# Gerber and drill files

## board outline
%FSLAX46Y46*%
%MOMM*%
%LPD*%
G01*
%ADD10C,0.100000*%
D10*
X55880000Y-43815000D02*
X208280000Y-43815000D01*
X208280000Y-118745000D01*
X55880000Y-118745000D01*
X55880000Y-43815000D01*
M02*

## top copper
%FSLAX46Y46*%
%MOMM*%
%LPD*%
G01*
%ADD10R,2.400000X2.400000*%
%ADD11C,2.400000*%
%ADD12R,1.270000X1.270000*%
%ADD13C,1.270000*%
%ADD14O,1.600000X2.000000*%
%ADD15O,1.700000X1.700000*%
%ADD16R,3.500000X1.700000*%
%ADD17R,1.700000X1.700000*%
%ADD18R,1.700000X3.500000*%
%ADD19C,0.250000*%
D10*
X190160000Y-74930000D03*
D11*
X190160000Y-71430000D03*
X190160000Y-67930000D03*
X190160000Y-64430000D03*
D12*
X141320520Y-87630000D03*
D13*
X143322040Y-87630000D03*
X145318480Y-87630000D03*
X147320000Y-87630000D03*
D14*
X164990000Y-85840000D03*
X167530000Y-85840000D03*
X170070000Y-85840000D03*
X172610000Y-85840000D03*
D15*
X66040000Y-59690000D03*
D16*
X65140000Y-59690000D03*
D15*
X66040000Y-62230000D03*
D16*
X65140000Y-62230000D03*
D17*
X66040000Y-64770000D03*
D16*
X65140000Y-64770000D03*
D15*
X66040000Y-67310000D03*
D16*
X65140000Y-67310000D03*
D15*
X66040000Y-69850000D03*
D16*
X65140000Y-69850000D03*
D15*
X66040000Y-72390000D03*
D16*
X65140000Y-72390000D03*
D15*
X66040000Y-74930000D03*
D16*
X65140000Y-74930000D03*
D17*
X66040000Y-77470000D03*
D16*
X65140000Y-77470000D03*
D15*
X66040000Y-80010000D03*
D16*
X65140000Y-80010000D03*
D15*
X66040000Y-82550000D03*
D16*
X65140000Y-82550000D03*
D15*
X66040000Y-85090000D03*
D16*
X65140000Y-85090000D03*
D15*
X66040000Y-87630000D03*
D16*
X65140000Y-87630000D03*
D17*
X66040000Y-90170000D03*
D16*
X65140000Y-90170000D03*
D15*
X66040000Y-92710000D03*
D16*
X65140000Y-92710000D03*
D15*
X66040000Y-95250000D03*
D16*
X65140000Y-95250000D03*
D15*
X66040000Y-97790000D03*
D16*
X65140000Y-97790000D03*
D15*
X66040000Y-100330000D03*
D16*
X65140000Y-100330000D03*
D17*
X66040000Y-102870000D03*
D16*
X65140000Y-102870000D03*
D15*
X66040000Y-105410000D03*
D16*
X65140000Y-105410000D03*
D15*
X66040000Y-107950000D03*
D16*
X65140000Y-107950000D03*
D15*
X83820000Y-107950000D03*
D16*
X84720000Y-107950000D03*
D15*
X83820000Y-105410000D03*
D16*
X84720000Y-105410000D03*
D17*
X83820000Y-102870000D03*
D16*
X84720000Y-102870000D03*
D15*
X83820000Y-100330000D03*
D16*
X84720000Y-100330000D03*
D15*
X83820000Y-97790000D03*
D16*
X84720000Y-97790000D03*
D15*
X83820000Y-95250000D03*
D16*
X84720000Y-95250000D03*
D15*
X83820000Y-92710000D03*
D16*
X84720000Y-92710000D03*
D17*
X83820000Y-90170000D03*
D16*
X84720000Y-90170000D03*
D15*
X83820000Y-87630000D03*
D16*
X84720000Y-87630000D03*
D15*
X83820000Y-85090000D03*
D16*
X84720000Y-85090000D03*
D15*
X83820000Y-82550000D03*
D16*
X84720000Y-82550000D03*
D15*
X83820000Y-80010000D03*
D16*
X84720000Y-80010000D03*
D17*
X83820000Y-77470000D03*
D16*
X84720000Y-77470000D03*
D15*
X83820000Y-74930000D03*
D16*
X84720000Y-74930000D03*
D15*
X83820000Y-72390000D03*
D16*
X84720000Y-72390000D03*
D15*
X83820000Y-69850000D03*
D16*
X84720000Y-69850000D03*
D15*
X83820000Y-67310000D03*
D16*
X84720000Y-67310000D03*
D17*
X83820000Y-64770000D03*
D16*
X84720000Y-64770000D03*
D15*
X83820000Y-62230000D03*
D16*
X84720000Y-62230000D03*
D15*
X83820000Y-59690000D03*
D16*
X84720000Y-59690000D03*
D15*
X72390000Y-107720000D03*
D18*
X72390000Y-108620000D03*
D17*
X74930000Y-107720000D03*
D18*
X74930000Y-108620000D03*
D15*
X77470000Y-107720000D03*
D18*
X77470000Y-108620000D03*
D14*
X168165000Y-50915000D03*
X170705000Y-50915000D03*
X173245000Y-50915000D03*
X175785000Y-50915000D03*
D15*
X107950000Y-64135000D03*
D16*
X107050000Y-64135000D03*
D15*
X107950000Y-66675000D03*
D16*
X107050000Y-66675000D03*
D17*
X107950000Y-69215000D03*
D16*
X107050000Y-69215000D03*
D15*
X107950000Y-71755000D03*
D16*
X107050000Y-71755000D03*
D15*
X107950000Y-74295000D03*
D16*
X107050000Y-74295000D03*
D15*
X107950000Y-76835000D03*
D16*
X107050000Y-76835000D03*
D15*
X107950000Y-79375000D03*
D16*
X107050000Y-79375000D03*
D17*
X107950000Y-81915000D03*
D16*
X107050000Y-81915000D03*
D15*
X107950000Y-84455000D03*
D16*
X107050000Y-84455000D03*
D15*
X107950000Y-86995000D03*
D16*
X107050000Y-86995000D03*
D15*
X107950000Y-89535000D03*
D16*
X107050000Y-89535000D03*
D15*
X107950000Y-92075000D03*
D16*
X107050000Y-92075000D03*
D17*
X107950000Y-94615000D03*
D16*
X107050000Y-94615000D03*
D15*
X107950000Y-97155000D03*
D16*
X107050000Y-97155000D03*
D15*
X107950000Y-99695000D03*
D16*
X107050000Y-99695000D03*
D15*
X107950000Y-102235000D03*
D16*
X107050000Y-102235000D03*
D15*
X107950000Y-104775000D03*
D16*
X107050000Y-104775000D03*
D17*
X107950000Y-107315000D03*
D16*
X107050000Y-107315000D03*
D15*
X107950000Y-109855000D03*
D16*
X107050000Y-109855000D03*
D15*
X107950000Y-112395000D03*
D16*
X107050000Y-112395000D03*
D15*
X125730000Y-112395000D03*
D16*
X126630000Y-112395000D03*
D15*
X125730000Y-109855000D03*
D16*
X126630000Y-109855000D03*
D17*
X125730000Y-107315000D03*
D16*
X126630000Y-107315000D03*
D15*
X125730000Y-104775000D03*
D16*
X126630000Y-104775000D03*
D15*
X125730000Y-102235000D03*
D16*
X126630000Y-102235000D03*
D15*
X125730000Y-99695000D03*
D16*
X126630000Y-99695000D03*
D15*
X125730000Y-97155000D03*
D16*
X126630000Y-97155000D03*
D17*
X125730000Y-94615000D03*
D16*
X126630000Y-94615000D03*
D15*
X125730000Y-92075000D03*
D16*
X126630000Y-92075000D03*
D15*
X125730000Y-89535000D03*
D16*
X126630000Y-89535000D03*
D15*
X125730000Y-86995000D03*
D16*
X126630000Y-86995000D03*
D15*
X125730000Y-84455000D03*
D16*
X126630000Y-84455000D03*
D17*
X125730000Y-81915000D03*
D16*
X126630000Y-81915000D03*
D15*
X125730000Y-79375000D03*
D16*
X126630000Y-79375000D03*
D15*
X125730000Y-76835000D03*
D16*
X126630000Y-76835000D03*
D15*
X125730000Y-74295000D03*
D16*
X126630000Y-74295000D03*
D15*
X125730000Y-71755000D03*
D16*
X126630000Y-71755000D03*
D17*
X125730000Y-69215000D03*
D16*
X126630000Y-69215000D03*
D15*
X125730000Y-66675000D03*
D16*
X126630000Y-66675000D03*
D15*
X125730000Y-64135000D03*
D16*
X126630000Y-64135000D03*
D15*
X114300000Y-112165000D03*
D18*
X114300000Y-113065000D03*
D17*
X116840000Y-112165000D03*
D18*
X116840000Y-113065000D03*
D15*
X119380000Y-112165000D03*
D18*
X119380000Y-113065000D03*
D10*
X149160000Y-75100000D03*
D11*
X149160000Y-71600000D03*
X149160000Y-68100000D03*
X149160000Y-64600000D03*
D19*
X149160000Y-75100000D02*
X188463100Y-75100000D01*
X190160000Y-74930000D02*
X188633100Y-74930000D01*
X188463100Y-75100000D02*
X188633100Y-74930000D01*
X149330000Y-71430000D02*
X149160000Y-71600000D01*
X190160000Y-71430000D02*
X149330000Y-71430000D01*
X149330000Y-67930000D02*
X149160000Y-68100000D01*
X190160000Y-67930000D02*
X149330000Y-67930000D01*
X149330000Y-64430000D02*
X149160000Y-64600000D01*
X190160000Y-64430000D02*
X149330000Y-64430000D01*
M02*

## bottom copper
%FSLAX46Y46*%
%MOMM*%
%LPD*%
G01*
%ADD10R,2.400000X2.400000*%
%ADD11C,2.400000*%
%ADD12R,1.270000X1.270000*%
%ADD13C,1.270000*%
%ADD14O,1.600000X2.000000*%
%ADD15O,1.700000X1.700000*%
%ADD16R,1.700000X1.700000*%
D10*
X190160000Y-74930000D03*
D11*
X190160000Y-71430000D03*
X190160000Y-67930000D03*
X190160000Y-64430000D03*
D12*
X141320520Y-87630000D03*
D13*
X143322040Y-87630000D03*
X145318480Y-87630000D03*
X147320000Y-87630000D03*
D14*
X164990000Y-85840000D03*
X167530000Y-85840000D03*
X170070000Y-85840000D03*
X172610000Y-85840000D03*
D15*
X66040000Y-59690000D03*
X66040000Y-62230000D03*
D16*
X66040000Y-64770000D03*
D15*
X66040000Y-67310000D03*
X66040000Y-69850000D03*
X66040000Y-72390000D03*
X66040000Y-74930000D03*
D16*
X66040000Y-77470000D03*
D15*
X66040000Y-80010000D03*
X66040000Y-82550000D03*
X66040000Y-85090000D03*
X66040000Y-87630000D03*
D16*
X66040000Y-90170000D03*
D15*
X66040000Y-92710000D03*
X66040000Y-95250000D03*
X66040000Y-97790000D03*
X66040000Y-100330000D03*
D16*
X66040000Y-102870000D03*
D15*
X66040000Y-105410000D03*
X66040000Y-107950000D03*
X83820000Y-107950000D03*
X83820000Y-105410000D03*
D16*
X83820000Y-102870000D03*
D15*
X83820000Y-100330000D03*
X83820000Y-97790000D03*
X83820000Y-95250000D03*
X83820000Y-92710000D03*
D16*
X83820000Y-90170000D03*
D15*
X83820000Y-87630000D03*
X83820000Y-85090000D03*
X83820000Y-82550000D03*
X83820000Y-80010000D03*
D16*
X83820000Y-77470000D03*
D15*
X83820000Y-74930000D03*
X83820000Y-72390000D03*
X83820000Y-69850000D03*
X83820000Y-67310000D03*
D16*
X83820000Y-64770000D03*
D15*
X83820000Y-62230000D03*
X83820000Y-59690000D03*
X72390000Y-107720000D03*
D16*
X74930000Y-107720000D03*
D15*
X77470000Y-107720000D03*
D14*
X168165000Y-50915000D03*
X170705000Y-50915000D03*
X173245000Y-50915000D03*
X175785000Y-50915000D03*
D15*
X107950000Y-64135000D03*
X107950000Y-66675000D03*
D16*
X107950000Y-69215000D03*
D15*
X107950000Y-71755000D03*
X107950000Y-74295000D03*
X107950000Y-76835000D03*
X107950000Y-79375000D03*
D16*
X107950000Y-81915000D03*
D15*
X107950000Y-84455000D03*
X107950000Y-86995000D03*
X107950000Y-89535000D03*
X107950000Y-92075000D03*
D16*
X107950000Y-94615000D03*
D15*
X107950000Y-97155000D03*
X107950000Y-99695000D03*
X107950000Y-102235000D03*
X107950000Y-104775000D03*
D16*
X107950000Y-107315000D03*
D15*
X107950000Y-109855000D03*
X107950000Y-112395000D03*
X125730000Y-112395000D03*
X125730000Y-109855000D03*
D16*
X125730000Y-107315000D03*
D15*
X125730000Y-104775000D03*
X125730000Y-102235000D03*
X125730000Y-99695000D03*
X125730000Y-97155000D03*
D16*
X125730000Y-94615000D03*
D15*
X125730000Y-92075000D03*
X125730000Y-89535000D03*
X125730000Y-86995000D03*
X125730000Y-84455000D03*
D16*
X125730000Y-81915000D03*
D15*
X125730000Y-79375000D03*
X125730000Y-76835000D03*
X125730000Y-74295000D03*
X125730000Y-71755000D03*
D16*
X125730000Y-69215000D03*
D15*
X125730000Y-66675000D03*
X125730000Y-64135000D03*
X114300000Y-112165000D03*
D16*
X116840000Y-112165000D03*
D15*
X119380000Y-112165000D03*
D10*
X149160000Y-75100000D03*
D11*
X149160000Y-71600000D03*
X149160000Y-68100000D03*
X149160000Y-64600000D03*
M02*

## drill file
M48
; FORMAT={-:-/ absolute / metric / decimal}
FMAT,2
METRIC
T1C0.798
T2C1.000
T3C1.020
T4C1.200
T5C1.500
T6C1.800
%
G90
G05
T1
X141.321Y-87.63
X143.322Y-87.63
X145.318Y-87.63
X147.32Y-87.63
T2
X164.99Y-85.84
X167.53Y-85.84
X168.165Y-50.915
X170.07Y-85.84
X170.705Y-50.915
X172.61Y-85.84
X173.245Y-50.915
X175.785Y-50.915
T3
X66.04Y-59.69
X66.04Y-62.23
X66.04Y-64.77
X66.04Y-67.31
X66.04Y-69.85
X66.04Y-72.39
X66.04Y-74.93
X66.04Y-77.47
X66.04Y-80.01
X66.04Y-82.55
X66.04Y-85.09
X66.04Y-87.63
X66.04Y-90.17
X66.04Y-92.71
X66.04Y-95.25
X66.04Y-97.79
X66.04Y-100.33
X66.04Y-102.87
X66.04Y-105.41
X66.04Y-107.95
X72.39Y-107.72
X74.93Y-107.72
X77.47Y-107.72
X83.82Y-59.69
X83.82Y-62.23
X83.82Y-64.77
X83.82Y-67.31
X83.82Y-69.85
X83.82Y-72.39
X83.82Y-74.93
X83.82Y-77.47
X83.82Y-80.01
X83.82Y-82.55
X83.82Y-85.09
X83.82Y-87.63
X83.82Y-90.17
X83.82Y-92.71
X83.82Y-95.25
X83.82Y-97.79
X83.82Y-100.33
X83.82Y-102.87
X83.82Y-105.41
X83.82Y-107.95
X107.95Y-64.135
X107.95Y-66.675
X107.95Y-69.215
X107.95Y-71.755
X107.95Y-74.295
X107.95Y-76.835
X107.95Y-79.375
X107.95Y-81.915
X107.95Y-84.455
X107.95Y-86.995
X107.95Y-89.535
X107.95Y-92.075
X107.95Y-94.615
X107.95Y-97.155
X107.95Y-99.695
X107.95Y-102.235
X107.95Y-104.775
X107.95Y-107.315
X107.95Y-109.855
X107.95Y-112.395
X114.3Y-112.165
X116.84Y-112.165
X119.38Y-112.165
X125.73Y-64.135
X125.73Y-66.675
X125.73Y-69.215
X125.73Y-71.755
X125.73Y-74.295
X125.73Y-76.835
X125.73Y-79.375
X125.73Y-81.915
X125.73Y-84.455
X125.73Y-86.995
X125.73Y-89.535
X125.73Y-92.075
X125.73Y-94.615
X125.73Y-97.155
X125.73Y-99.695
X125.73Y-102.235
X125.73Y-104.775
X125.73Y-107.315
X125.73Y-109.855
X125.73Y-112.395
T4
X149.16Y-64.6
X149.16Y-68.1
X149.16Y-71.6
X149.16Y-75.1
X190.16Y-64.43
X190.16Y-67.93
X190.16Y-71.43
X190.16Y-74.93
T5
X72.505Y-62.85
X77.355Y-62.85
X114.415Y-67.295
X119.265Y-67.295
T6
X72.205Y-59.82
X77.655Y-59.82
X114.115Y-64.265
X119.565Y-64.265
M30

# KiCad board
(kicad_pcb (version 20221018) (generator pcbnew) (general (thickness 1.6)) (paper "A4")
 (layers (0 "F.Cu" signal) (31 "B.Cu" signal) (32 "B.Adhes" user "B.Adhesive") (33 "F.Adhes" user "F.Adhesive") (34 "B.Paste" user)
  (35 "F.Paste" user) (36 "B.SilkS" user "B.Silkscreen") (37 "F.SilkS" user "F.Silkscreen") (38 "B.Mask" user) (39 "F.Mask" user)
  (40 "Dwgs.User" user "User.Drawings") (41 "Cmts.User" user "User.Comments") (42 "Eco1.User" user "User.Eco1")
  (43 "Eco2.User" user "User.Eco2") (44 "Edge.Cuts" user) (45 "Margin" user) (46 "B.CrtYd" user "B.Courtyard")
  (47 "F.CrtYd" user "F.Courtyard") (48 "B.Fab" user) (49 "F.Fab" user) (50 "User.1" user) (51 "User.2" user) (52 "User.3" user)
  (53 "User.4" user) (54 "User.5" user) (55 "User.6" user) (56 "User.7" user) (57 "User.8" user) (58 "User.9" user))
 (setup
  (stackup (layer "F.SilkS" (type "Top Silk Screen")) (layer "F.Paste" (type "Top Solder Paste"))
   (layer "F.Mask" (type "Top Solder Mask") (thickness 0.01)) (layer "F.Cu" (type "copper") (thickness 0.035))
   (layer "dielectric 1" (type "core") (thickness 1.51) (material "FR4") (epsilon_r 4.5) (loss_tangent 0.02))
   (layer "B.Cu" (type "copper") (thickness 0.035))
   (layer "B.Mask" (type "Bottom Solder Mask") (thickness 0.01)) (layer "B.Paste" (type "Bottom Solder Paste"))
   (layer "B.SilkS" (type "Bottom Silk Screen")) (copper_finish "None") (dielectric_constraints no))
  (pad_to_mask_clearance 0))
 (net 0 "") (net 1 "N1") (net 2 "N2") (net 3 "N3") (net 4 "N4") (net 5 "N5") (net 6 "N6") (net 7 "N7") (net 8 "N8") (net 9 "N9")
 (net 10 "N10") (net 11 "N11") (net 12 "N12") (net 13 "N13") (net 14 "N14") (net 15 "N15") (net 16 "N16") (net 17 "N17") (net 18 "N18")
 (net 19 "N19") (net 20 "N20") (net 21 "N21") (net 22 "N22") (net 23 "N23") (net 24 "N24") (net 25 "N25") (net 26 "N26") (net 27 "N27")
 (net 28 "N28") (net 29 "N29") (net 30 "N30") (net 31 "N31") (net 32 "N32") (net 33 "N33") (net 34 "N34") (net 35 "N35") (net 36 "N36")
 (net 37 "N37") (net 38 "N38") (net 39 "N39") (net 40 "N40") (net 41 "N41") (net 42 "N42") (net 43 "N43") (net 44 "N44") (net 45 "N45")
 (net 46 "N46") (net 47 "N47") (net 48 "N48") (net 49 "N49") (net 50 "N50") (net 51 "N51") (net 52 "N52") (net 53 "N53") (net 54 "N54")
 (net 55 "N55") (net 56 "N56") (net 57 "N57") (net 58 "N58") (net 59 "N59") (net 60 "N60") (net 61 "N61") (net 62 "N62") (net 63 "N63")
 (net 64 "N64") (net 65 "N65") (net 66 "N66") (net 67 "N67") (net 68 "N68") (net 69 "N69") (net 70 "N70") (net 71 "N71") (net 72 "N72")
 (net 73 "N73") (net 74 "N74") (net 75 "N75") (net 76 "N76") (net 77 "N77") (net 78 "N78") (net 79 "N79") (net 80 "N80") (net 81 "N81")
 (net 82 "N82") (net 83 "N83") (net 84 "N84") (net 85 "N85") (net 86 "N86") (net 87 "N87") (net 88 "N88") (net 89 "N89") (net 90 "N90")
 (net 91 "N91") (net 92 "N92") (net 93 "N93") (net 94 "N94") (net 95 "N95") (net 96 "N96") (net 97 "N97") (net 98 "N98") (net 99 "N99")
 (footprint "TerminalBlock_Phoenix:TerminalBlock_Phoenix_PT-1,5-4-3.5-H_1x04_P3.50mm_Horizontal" (layer "F.Cu") (at 190.16 74.93 90)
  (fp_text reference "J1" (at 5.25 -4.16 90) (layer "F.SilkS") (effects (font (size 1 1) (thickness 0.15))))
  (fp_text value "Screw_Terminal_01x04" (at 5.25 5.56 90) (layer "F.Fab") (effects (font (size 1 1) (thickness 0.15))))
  (pad "1" thru_hole rect (at 0 0 90) (size 2.4 2.4) (drill 1.2) (layers "*.Cu" "*.Mask") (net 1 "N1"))
  (pad "2" thru_hole circle (at 3.5 0 90) (size 2.4 2.4) (drill 1.2) (layers "*.Cu" "*.Mask") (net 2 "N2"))
  (pad "3" thru_hole circle (at 7 0 90) (size 2.4 2.4) (drill 1.2) (layers "*.Cu" "*.Mask") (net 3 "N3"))
  (pad "4" thru_hole circle (at 10.5 0 90) (size 2.4 2.4) (drill 1.2) (layers "*.Cu" "*.Mask") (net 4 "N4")))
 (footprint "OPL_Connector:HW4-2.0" (layer "F.Cu") (at 144.32026 87.63)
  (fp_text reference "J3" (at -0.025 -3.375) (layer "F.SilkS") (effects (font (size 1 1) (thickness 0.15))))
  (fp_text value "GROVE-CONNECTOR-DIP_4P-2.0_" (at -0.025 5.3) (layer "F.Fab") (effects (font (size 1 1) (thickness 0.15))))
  (pad "1" thru_hole rect (at -2.99974 0) (size 1.27 1.27) (drill 0.79756) (layers "*.Cu" "*.Mask") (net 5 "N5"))
  (pad "2" thru_hole circle (at -0.99822 0) (size 1.27 1.27) (drill 0.79756) (layers "*.Cu" "*.Mask") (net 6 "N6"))
  (pad "3" thru_hole circle (at 0.99822 0) (size 1.27 1.27) (drill 0.79756) (layers "*.Cu" "*.Mask") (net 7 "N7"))
  (pad "4" thru_hole circle (at 2.99974 0) (size 1.27 1.27) (drill 0.79756) (layers "*.Cu" "*.Mask") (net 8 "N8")))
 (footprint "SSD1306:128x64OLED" (layer "F.Cu") (at 168.61 96.44)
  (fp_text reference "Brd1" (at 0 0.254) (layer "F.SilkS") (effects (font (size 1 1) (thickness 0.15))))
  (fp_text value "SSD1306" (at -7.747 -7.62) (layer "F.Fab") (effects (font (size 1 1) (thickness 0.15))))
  (pad "1" thru_hole oval (at -3.62 -10.6 90) (size 2 1.6) (drill 1) (layers "*.Cu" "*.Mask") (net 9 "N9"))
  (pad "2" thru_hole oval (at -1.08 -10.6 90) (size 2 1.6) (drill 1) (layers "*.Cu" "*.Mask") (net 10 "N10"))
  (pad "3" thru_hole oval (at 1.46 -10.6 90) (size 2 1.6) (drill 1) (layers "*.Cu" "*.Mask") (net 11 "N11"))
  (pad "4" thru_hole oval (at 4 -10.6 90) (size 2 1.6) (drill 1) (layers "*.Cu" "*.Mask") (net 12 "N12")))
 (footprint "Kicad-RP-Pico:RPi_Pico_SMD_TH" (layer "F.Cu") (at 74.93 83.82)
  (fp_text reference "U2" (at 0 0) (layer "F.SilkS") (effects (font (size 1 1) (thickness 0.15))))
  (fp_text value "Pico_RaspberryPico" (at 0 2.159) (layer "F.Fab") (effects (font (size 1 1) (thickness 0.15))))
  (pad "" np_thru_hole oval (at -2.725 -24) (size 1.8 1.8) (drill 1.8) (layers "*.Cu" "*.Mask"))
  (pad "" np_thru_hole oval (at -2.425 -20.97) (size 1.5 1.5) (drill 1.5) (layers "*.Cu" "*.Mask"))
  (pad "" np_thru_hole oval (at 2.425 -20.97) (size 1.5 1.5) (drill 1.5) (layers "*.Cu" "*.Mask"))
  (pad "" np_thru_hole oval (at 2.725 -24) (size 1.8 1.8) (drill 1.8) (layers "*.Cu" "*.Mask"))
  (pad "1" thru_hole oval (at -8.89 -24.13) (size 1.7 1.7) (drill 1.02) (layers "*.Cu" "*.Mask") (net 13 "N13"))
  (pad "1" smd rect (at -8.89 -24.13) (size 3.5 1.7) (drill (offset -0.9 0)) (layers "F.Cu" "F.Mask") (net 13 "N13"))
  (pad "2" thru_hole oval (at -8.89 -21.59) (size 1.7 1.7) (drill 1.02) (layers "*.Cu" "*.Mask") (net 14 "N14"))
  (pad "2" smd rect (at -8.89 -21.59) (size 3.5 1.7) (drill (offset -0.9 0)) (layers "F.Cu" "F.Mask") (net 14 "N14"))
  (pad "3" thru_hole rect (at -8.89 -19.05) (size 1.7 1.7) (drill 1.02) (layers "*.Cu" "*.Mask") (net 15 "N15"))
  (pad "3" smd rect (at -8.89 -19.05) (size 3.5 1.7) (drill (offset -0.9 0)) (layers "F.Cu" "F.Mask") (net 15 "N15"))
  (pad "4" thru_hole oval (at -8.89 -16.51) (size 1.7 1.7) (drill 1.02) (layers "*.Cu" "*.Mask") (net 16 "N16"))
  (pad "4" smd rect (at -8.89 -16.51) (size 3.5 1.7) (drill (offset -0.9 0)) (layers "F.Cu" "F.Mask") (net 16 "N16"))
  (pad "5" thru_hole oval (at -8.89 -13.97) (size 1.7 1.7) (drill 1.02) (layers "*.Cu" "*.Mask") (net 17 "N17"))
  (pad "5" smd rect (at -8.89 -13.97) (size 3.5 1.7) (drill (offset -0.9 0)) (layers "F.Cu" "F.Mask") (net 17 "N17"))
  (pad "6" thru_hole oval (at -8.89 -11.43) (size 1.7 1.7) (drill 1.02) (layers "*.Cu" "*.Mask") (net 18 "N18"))
  (pad "6" smd rect (at -8.89 -11.43) (size 3.5 1.7) (drill (offset -0.9 0)) (layers "F.Cu" "F.Mask") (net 18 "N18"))
  (pad "7" thru_hole oval (at -8.89 -8.89) (size 1.7 1.7) (drill 1.02) (layers "*.Cu" "*.Mask") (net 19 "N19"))
  (pad "7" smd rect (at -8.89 -8.89) (size 3.5 1.7) (drill (offset -0.9 0)) (layers "F.Cu" "F.Mask") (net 19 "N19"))
  (pad "8" thru_hole rect (at -8.89 -6.35) (size 1.7 1.7) (drill 1.02) (layers "*.Cu" "*.Mask") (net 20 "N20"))
  (pad "8" smd rect (at -8.89 -6.35) (size 3.5 1.7) (drill (offset -0.9 0)) (layers "F.Cu" "F.Mask") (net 20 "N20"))
  (pad "9" thru_hole oval (at -8.89 -3.81) (size 1.7 1.7) (drill 1.02) (layers "*.Cu" "*.Mask") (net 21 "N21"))
  (pad "9" smd rect (at -8.89 -3.81) (size 3.5 1.7) (drill (offset -0.9 0)) (layers "F.Cu" "F.Mask") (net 21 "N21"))
  (pad "10" thru_hole oval (at -8.89 -1.27) (size 1.7 1.7) (drill 1.02) (layers "*.Cu" "*.Mask") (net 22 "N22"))
  (pad "10" smd rect (at -8.89 -1.27) (size 3.5 1.7) (drill (offset -0.9 0)) (layers "F.Cu" "F.Mask") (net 22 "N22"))
  (pad "11" thru_hole oval (at -8.89 1.27) (size 1.7 1.7) (drill 1.02) (layers "*.Cu" "*.Mask") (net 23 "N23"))
  (pad "11" smd rect (at -8.89 1.27) (size 3.5 1.7) (drill (offset -0.9 0)) (layers "F.Cu" "F.Mask") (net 23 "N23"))
  (pad "12" thru_hole oval (at -8.89 3.81) (size 1.7 1.7) (drill 1.02) (layers "*.Cu" "*.Mask") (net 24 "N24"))
  (pad "12" smd rect (at -8.89 3.81) (size 3.5 1.7) (drill (offset -0.9 0)) (layers "F.Cu" "F.Mask") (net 24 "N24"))
  (pad "13" thru_hole rect (at -8.89 6.35) (size 1.7 1.7) (drill 1.02) (layers "*.Cu" "*.Mask") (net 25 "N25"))
  (pad "13" smd rect (at -8.89 6.35) (size 3.5 1.7) (drill (offset -0.9 0)) (layers "F.Cu" "F.Mask") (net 25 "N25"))
  (pad "14" thru_hole oval (at -8.89 8.89) (size 1.7 1.7) (drill 1.02) (layers "*.Cu" "*.Mask") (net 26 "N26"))
  (pad "14" smd rect (at -8.89 8.89) (size 3.5 1.7) (drill (offset -0.9 0)) (layers "F.Cu" "F.Mask") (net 26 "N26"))
  (pad "15" thru_hole oval (at -8.89 11.43) (size 1.7 1.7) (drill 1.02) (layers "*.Cu" "*.Mask") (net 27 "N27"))
  (pad "15" smd rect (at -8.89 11.43) (size 3.5 1.7) (drill (offset -0.9 0)) (layers "F.Cu" "F.Mask") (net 27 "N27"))
  (pad "16" thru_hole oval (at -8.89 13.97) (size 1.7 1.7) (drill 1.02) (layers "*.Cu" "*.Mask") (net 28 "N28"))
  (pad "16" smd rect (at -8.89 13.97) (size 3.5 1.7) (drill (offset -0.9 0)) (layers "F.Cu" "F.Mask") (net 28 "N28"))
  (pad "17" thru_hole oval (at -8.89 16.51) (size 1.7 1.7) (drill 1.02) (layers "*.Cu" "*.Mask") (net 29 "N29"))
  (pad "17" smd rect (at -8.89 16.51) (size 3.5 1.7) (drill (offset -0.9 0)) (layers "F.Cu" "F.Mask") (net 29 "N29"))
  (pad "18" thru_hole rect (at -8.89 19.05) (size 1.7 1.7) (drill 1.02) (layers "*.Cu" "*.Mask") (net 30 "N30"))
  (pad "18" smd rect (at -8.89 19.05) (size 3.5 1.7) (drill (offset -0.9 0)) (layers "F.Cu" "F.Mask") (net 30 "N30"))
  (pad "19" thru_hole oval (at -8.89 21.59) (size 1.7 1.7) (drill 1.02) (layers "*.Cu" "*.Mask") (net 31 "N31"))
  (pad "19" smd rect (at -8.89 21.59) (size 3.5 1.7) (drill (offset -0.9 0)) (layers "F.Cu" "F.Mask") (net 31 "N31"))
  (pad "20" thru_hole oval (at -8.89 24.13) (size 1.7 1.7) (drill 1.02) (layers "*.Cu" "*.Mask") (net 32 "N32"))
  (pad "20" smd rect (at -8.89 24.13) (size 3.5 1.7) (drill (offset -0.9 0)) (layers "F.Cu" "F.Mask") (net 32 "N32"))
  (pad "21" thru_hole oval (at 8.89 24.13) (size 1.7 1.7) (drill 1.02) (layers "*.Cu" "*.Mask") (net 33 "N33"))
  (pad "21" smd rect (at 8.89 24.13) (size 3.5 1.7) (drill (offset 0.9 0)) (layers "F.Cu" "F.Mask") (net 33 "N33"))
  (pad "22" thru_hole oval (at 8.89 21.59) (size 1.7 1.7) (drill 1.02) (layers "*.Cu" "*.Mask") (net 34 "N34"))
  (pad "22" smd rect (at 8.89 21.59) (size 3.5 1.7) (drill (offset 0.9 0)) (layers "F.Cu" "F.Mask") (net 34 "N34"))
  (pad "23" thru_hole rect (at 8.89 19.05) (size 1.7 1.7) (drill 1.02) (layers "*.Cu" "*.Mask") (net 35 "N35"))
  (pad "23" smd rect (at 8.89 19.05) (size 3.5 1.7) (drill (offset 0.9 0)) (layers "F.Cu" "F.Mask") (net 35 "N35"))
  (pad "24" thru_hole oval (at 8.89 16.51) (size 1.7 1.7) (drill 1.02) (layers "*.Cu" "*.Mask") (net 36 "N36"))
  (pad "24" smd rect (at 8.89 16.51) (size 3.5 1.7) (drill (offset 0.9 0)) (layers "F.Cu" "F.Mask") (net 36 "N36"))
  (pad "25" thru_hole oval (at 8.89 13.97) (size 1.7 1.7) (drill 1.02) (layers "*.Cu" "*.Mask") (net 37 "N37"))
  (pad "25" smd rect (at 8.89 13.97) (size 3.5 1.7) (drill (offset 0.9 0)) (layers "F.Cu" "F.Mask") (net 37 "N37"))
  (pad "26" thru_hole oval (at 8.89 11.43) (size 1.7 1.7) (drill 1.02) (layers "*.Cu" "*.Mask") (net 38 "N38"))
  (pad "26" smd rect (at 8.89 11.43) (size 3.5 1.7) (drill (offset 0.9 0)) (layers "F.Cu" "F.Mask") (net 38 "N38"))
  (pad "27" thru_hole oval (at 8.89 8.89) (size 1.7 1.7) (drill 1.02) (layers "*.Cu" "*.Mask") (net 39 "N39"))
  (pad "27" smd rect (at 8.89 8.89) (size 3.5 1.7) (drill (offset 0.9 0)) (layers "F.Cu" "F.Mask") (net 39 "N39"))
  (pad "28" thru_hole rect (at 8.89 6.35) (size 1.7 1.7) (drill 1.02) (layers "*.Cu" "*.Mask") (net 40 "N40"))
  (pad "28" smd rect (at 8.89 6.35) (size 3.5 1.7) (drill (offset 0.9 0)) (layers "F.Cu" "F.Mask") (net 40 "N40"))
  (pad "29" thru_hole oval (at 8.89 3.81) (size 1.7 1.7) (drill 1.02) (layers "*.Cu" "*.Mask") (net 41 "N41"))
  (pad "29" smd rect (at 8.89 3.81) (size 3.5 1.7) (drill (offset 0.9 0)) (layers "F.Cu" "F.Mask") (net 41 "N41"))
  (pad "30" thru_hole oval (at 8.89 1.27) (size 1.7 1.7) (drill 1.02) (layers "*.Cu" "*.Mask") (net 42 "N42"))
  (pad "30" smd rect (at 8.89 1.27) (size 3.5 1.7) (drill (offset 0.9 0)) (layers "F.Cu" "F.Mask") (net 42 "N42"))
  (pad "31" thru_hole oval (at 8.89 -1.27) (size 1.7 1.7) (drill 1.02) (layers "*.Cu" "*.Mask") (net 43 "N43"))
  (pad "31" smd rect (at 8.89 -1.27) (size 3.5 1.7) (drill (offset 0.9 0)) (layers "F.Cu" "F.Mask") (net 43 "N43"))
  (pad "32" thru_hole oval (at 8.89 -3.81) (size 1.7 1.7) (drill 1.02) (layers "*.Cu" "*.Mask") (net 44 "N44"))
  (pad "32" smd rect (at 8.89 -3.81) (size 3.5 1.7) (drill (offset 0.9 0)) (layers "F.Cu" "F.Mask") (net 44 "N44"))
  (pad "33" thru_hole rect (at 8.89 -6.35) (size 1.7 1.7) (drill 1.02) (layers "*.Cu" "*.Mask") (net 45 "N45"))
  (pad "33" smd rect (at 8.89 -6.35) (size 3.5 1.7) (drill (offset 0.9 0)) (layers "F.Cu" "F.Mask") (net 45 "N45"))
  (pad "34" thru_hole oval (at 8.89 -8.89) (size 1.7 1.7) (drill 1.02) (layers "*.Cu" "*.Mask") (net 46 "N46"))
  (pad "34" smd rect (at 8.89 -8.89) (size 3.5 1.7) (drill (offset 0.9 0)) (layers "F.Cu" "F.Mask") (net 46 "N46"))
  (pad "35" thru_hole oval (at 8.89 -11.43) (size 1.7 1.7) (drill 1.02) (layers "*.Cu" "*.Mask") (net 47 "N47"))
  (pad "35" smd rect (at 8.89 -11.43) (size 3.5 1.7) (drill (offset 0.9 0)) (layers "F.Cu" "F.Mask") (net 47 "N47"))
  (pad "36" thru_hole oval (at 8.89 -13.97) (size 1.7 1.7) (drill 1.02) (layers "*.Cu" "*.Mask") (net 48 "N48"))
  (pad "36" smd rect (at 8.89 -13.97) (size 3.5 1.7) (drill (offset 0.9 0)) (layers "F.Cu" "F.Mask") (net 48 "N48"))
  (pad "37" thru_hole oval (at 8.89 -16.51) (size 1.7 1.7) (drill 1.02) (layers "*.Cu" "*.Mask") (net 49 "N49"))
  (pad "37" smd rect (at 8.89 -16.51) (size 3.5 1.7) (drill (offset 0.9 0)) (layers "F.Cu" "F.Mask") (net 49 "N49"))
  (pad "38" thru_hole rect (at 8.89 -19.05) (size 1.7 1.7) (drill 1.02) (layers "*.Cu" "*.Mask") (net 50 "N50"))
  (pad "38" smd rect (at 8.89 -19.05) (size 3.5 1.7) (drill (offset 0.9 0)) (layers "F.Cu" "F.Mask") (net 50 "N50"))
  (pad "39" thru_hole oval (at 8.89 -21.59) (size 1.7 1.7) (drill 1.02) (layers "*.Cu" "*.Mask") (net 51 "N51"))
  (pad "39" smd rect (at 8.89 -21.59) (size 3.5 1.7) (drill (offset 0.9 0)) (layers "F.Cu" "F.Mask") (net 51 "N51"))
  (pad "40" thru_hole oval (at 8.89 -24.13) (size 1.7 1.7) (drill 1.02) (layers "*.Cu" "*.Mask") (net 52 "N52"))
  (pad "40" smd rect (at 8.89 -24.13) (size 3.5 1.7) (drill (offset 0.9 0)) (layers "F.Cu" "F.Mask") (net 52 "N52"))
  (pad "41" thru_hole oval (at -2.54 23.9) (size 1.7 1.7) (drill 1.02) (layers "*.Cu" "*.Mask"))
  (pad "41" smd rect (at -2.54 23.9 90) (size 3.5 1.7) (drill (offset -0.9 0)) (layers "F.Cu" "F.Mask"))
  (pad "42" thru_hole rect (at 0 23.9) (size 1.7 1.7) (drill 1.02) (layers "*.Cu" "*.Mask"))
  (pad "42" smd rect (at 0 23.9 90) (size 3.5 1.7) (drill (offset -0.9 0)) (layers "F.Cu" "F.Mask"))
  (pad "43" thru_hole oval (at 2.54 23.9) (size 1.7 1.7) (drill 1.02) (layers "*.Cu" "*.Mask"))
  (pad "43" smd rect (at 2.54 23.9 90) (size 3.5 1.7) (drill (offset -0.9 0)) (layers "F.Cu" "F.Mask")))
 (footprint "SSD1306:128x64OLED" (layer "F.Cu") (at 171.785 61.515)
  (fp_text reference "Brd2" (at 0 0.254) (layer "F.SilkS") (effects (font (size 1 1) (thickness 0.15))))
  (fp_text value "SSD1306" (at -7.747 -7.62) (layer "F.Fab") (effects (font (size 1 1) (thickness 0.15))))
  (pad "1" thru_hole oval (at -3.62 -10.6 90) (size 2 1.6) (drill 1) (layers "*.Cu" "*.Mask") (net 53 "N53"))
  (pad "2" thru_hole oval (at -1.08 -10.6 90) (size 2 1.6) (drill 1) (layers "*.Cu" "*.Mask") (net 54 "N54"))
  (pad "3" thru_hole oval (at 1.46 -10.6 90) (size 2 1.6) (drill 1) (layers "*.Cu" "*.Mask") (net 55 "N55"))
  (pad "4" thru_hole oval (at 4 -10.6 90) (size 2 1.6) (drill 1) (layers "*.Cu" "*.Mask") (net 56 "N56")))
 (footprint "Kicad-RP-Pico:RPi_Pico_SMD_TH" (layer "F.Cu") (at 116.84 88.265)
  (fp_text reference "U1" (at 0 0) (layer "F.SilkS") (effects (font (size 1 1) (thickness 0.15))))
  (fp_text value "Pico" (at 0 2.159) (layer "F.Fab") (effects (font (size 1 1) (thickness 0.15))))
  (pad "" np_thru_hole oval (at -2.725 -24) (size 1.8 1.8) (drill 1.8) (layers "*.Cu" "*.Mask"))
  (pad "" np_thru_hole oval (at -2.425 -20.97) (size 1.5 1.5) (drill 1.5) (layers "*.Cu" "*.Mask"))
  (pad "" np_thru_hole oval (at 2.425 -20.97) (size 1.5 1.5) (drill 1.5) (layers "*.Cu" "*.Mask"))
  (pad "" np_thru_hole oval (at 2.725 -24) (size 1.8 1.8) (drill 1.8) (layers "*.Cu" "*.Mask"))
  (pad "1" thru_hole oval (at -8.89 -24.13) (size 1.7 1.7) (drill 1.02) (layers "*.Cu" "*.Mask") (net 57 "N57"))
  (pad "1" smd rect (at -8.89 -24.13) (size 3.5 1.7) (drill (offset -0.9 0)) (layers "F.Cu" "F.Mask") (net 57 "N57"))
  (pad "2" thru_hole oval (at -8.89 -21.59) (size 1.7 1.7) (drill 1.02) (layers "*.Cu" "*.Mask") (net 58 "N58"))
  (pad "2" smd rect (at -8.89 -21.59) (size 3.5 1.7) (drill (offset -0.9 0)) (layers "F.Cu" "F.Mask") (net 58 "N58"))
  (pad "3" thru_hole rect (at -8.89 -19.05) (size 1.7 1.7) (drill 1.02) (layers "*.Cu" "*.Mask") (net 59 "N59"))
  (pad "3" smd rect (at -8.89 -19.05) (size 3.5 1.7) (drill (offset -0.9 0)) (layers "F.Cu" "F.Mask") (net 59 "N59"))
  (pad "4" thru_hole oval (at -8.89 -16.51) (size 1.7 1.7) (drill 1.02) (layers "*.Cu" "*.Mask") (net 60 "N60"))
  (pad "4" smd rect (at -8.89 -16.51) (size 3.5 1.7) (drill (offset -0.9 0)) (layers "F.Cu" "F.Mask") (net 60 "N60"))
  (pad "5" thru_hole oval (at -8.89 -13.97) (size 1.7 1.7) (drill 1.02) (layers "*.Cu" "*.Mask") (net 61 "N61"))
  (pad "5" smd rect (at -8.89 -13.97) (size 3.5 1.7) (drill (offset -0.9 0)) (layers "F.Cu" "F.Mask") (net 61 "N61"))
  (pad "6" thru_hole oval (at -8.89 -11.43) (size 1.7 1.7) (drill 1.02) (layers "*.Cu" "*.Mask") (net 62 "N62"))
  (pad "6" smd rect (at -8.89 -11.43) (size 3.5 1.7) (drill (offset -0.9 0)) (layers "F.Cu" "F.Mask") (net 62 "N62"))
  (pad "7" thru_hole oval (at -8.89 -8.89) (size 1.7 1.7) (drill 1.02) (layers "*.Cu" "*.Mask") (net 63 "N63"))
  (pad "7" smd rect (at -8.89 -8.89) (size 3.5 1.7) (drill (offset -0.9 0)) (layers "F.Cu" "F.Mask") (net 63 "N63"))
  (pad "8" thru_hole rect (at -8.89 -6.35) (size 1.7 1.7) (drill 1.02) (layers "*.Cu" "*.Mask") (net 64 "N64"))
  (pad "8" smd rect (at -8.89 -6.35) (size 3.5 1.7) (drill (offset -0.9 0)) (layers "F.Cu" "F.Mask") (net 64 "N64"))
  (pad "9" thru_hole oval (at -8.89 -3.81) (size 1.7 1.7) (drill 1.02) (layers "*.Cu" "*.Mask") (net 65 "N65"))
  (pad "9" smd rect (at -8.89 -3.81) (size 3.5 1.7) (drill (offset -0.9 0)) (layers "F.Cu" "F.Mask") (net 65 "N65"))
  (pad "10" thru_hole oval (at -8.89 -1.27) (size 1.7 1.7) (drill 1.02) (layers "*.Cu" "*.Mask") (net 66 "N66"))
  (pad "10" smd rect (at -8.89 -1.27) (size 3.5 1.7) (drill (offset -0.9 0)) (layers "F.Cu" "F.Mask") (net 66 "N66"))
  (pad "11" thru_hole oval (at -8.89 1.27) (size 1.7 1.7) (drill 1.02) (layers "*.Cu" "*.Mask") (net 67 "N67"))
  (pad "11" smd rect (at -8.89 1.27) (size 3.5 1.7) (drill (offset -0.9 0)) (layers "F.Cu" "F.Mask") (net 67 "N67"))
  (pad "12" thru_hole oval (at -8.89 3.81) (size 1.7 1.7) (drill 1.02) (layers "*.Cu" "*.Mask") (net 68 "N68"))
  (pad "12" smd rect (at -8.89 3.81) (size 3.5 1.7) (drill (offset -0.9 0)) (layers "F.Cu" "F.Mask") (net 68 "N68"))
  (pad "13" thru_hole rect (at -8.89 6.35) (size 1.7 1.7) (drill 1.02) (layers "*.Cu" "*.Mask") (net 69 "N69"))
  (pad "13" smd rect (at -8.89 6.35) (size 3.5 1.7) (drill (offset -0.9 0)) (layers "F.Cu" "F.Mask") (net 69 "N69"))
  (pad "14" thru_hole oval (at -8.89 8.89) (size 1.7 1.7) (drill 1.02) (layers "*.Cu" "*.Mask") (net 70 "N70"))
  (pad "14" smd rect (at -8.89 8.89) (size 3.5 1.7) (drill (offset -0.9 0)) (layers "F.Cu" "F.Mask") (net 70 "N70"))
  (pad "15" thru_hole oval (at -8.89 11.43) (size 1.7 1.7) (drill 1.02) (layers "*.Cu" "*.Mask") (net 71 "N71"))
  (pad "15" smd rect (at -8.89 11.43) (size 3.5 1.7) (drill (offset -0.9 0)) (layers "F.Cu" "F.Mask") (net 71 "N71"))
  (pad "16" thru_hole oval (at -8.89 13.97) (size 1.7 1.7) (drill 1.02) (layers "*.Cu" "*.Mask") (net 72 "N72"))
  (pad "16" smd rect (at -8.89 13.97) (size 3.5 1.7) (drill (offset -0.9 0)) (layers "F.Cu" "F.Mask") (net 72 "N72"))
  (pad "17" thru_hole oval (at -8.89 16.51) (size 1.7 1.7) (drill 1.02) (layers "*.Cu" "*.Mask") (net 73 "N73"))
  (pad "17" smd rect (at -8.89 16.51) (size 3.5 1.7) (drill (offset -0.9 0)) (layers "F.Cu" "F.Mask") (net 73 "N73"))
  (pad "18" thru_hole rect (at -8.89 19.05) (size 1.7 1.7) (drill 1.02) (layers "*.Cu" "*.Mask") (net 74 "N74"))
  (pad "18" smd rect (at -8.89 19.05) (size 3.5 1.7) (drill (offset -0.9 0)) (layers "F.Cu" "F.Mask") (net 74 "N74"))
  (pad "19" thru_hole oval (at -8.89 21.59) (size 1.7 1.7) (drill 1.02) (layers "*.Cu" "*.Mask") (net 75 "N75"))
  (pad "19" smd rect (at -8.89 21.59) (size 3.5 1.7) (drill (offset -0.9 0)) (layers "F.Cu" "F.Mask") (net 75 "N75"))
  (pad "20" thru_hole oval (at -8.89 24.13) (size 1.7 1.7) (drill 1.02) (layers "*.Cu" "*.Mask") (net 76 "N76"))
  (pad "20" smd rect (at -8.89 24.13) (size 3.5 1.7) (drill (offset -0.9 0)) (layers "F.Cu" "F.Mask") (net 76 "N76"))
  (pad "21" thru_hole oval (at 8.89 24.13) (size 1.7 1.7) (drill 1.02) (layers "*.Cu" "*.Mask") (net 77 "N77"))
  (pad "21" smd rect (at 8.89 24.13) (size 3.5 1.7) (drill (offset 0.9 0)) (layers "F.Cu" "F.Mask") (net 77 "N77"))
  (pad "22" thru_hole oval (at 8.89 21.59) (size 1.7 1.7) (drill 1.02) (layers "*.Cu" "*.Mask") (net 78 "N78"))
  (pad "22" smd rect (at 8.89 21.59) (size 3.5 1.7) (drill (offset 0.9 0)) (layers "F.Cu" "F.Mask") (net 78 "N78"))
  (pad "23" thru_hole rect (at 8.89 19.05) (size 1.7 1.7) (drill 1.02) (layers "*.Cu" "*.Mask") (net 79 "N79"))
  (pad "23" smd rect (at 8.89 19.05) (size 3.5 1.7) (drill (offset 0.9 0)) (layers "F.Cu" "F.Mask") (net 79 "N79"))
  (pad "24" thru_hole oval (at 8.89 16.51) (size 1.7 1.7) (drill 1.02) (layers "*.Cu" "*.Mask") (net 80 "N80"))
  (pad "24" smd rect (at 8.89 16.51) (size 3.5 1.7) (drill (offset 0.9 0)) (layers "F.Cu" "F.Mask") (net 80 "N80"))
  (pad "25" thru_hole oval (at 8.89 13.97) (size 1.7 1.7) (drill 1.02) (layers "*.Cu" "*.Mask") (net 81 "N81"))
  (pad "25" smd rect (at 8.89 13.97) (size 3.5 1.7) (drill (offset 0.9 0)) (layers "F.Cu" "F.Mask") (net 81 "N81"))
  (pad "26" thru_hole oval (at 8.89 11.43) (size 1.7 1.7) (drill 1.02) (layers "*.Cu" "*.Mask") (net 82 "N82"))
  (pad "26" smd rect (at 8.89 11.43) (size 3.5 1.7) (drill (offset 0.9 0)) (layers "F.Cu" "F.Mask") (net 82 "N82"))
  (pad "27" thru_hole oval (at 8.89 8.89) (size 1.7 1.7) (drill 1.02) (layers "*.Cu" "*.Mask") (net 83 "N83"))
  (pad "27" smd rect (at 8.89 8.89) (size 3.5 1.7) (drill (offset 0.9 0)) (layers "F.Cu" "F.Mask") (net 83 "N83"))
  (pad "28" thru_hole rect (at 8.89 6.35) (size 1.7 1.7) (drill 1.02) (layers "*.Cu" "*.Mask") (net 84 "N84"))
  (pad "28" smd rect (at 8.89 6.35) (size 3.5 1.7) (drill (offset 0.9 0)) (layers "F.Cu" "F.Mask") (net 84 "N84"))
  (pad "29" thru_hole oval (at 8.89 3.81) (size 1.7 1.7) (drill 1.02) (layers "*.Cu" "*.Mask") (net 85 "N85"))
  (pad "29" smd rect (at 8.89 3.81) (size 3.5 1.7) (drill (offset 0.9 0)) (layers "F.Cu" "F.Mask") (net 85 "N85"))
  (pad "30" thru_hole oval (at 8.89 1.27) (size 1.7 1.7) (drill 1.02) (layers "*.Cu" "*.Mask") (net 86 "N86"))
  (pad "30" smd rect (at 8.89 1.27) (size 3.5 1.7) (drill (offset 0.9 0)) (layers "F.Cu" "F.Mask") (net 86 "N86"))
  (pad "31" thru_hole oval (at 8.89 -1.27) (size 1.7 1.7) (drill 1.02) (layers "*.Cu" "*.Mask") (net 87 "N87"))
  (pad "31" smd rect (at 8.89 -1.27) (size 3.5 1.7) (drill (offset 0.9 0)) (layers "F.Cu" "F.Mask") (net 87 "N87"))
  (pad "32" thru_hole oval (at 8.89 -3.81) (size 1.7 1.7) (drill 1.02) (layers "*.Cu" "*.Mask") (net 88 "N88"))
  (pad "32" smd rect (at 8.89 -3.81) (size 3.5 1.7) (drill (offset 0.9 0)) (layers "F.Cu" "F.Mask") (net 88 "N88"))
  (pad "33" thru_hole rect (at 8.89 -6.35) (size 1.7 1.7) (drill 1.02) (layers "*.Cu" "*.Mask") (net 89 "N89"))
  (pad "33" smd rect (at 8.89 -6.35) (size 3.5 1.7) (drill (offset 0.9 0)) (layers "F.Cu" "F.Mask") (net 89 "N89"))
  (pad "34" thru_hole oval (at 8.89 -8.89) (size 1.7 1.7) (drill 1.02) (layers "*.Cu" "*.Mask") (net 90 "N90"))
  (pad "34" smd rect (at 8.89 -8.89) (size 3.5 1.7) (drill (offset 0.9 0)) (layers "F.Cu" "F.Mask") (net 90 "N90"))
  (pad "35" thru_hole oval (at 8.89 -11.43) (size 1.7 1.7) (drill 1.02) (layers "*.Cu" "*.Mask") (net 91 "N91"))
  (pad "35" smd rect (at 8.89 -11.43) (size 3.5 1.7) (drill (offset 0.9 0)) (layers "F.Cu" "F.Mask") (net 91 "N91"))
  (pad "36" thru_hole oval (at 8.89 -13.97) (size 1.7 1.7) (drill 1.02) (layers "*.Cu" "*.Mask") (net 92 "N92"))
  (pad "36" smd rect (at 8.89 -13.97) (size 3.5 1.7) (drill (offset 0.9 0)) (layers "F.Cu" "F.Mask") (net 92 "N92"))
  (pad "37" thru_hole oval (at 8.89 -16.51) (size 1.7 1.7) (drill 1.02) (layers "*.Cu" "*.Mask") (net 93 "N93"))
  (pad "37" smd rect (at 8.89 -16.51) (size 3.5 1.7) (drill (offset 0.9 0)) (layers "F.Cu" "F.Mask") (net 93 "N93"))
  (pad "38" thru_hole rect (at 8.89 -19.05) (size 1.7 1.7) (drill 1.02) (layers "*.Cu" "*.Mask") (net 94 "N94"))
  (pad "38" smd rect (at 8.89 -19.05) (size 3.5 1.7) (drill (offset 0.9 0)) (layers "F.Cu" "F.Mask") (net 94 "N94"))
  (pad "39" thru_hole oval (at 8.89 -21.59) (size 1.7 1.7) (drill 1.02) (layers "*.Cu" "*.Mask") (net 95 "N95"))
  (pad "39" smd rect (at 8.89 -21.59) (size 3.5 1.7) (drill (offset 0.9 0)) (layers "F.Cu" "F.Mask") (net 95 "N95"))
  (pad "40" thru_hole oval (at 8.89 -24.13) (size 1.7 1.7) (drill 1.02) (layers "*.Cu" "*.Mask") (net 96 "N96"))
  (pad "40" smd rect (at 8.89 -24.13) (size 3.5 1.7) (drill (offset 0.9 0)) (layers "F.Cu" "F.Mask") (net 96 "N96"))
  (pad "41" thru_hole oval (at -2.54 23.9) (size 1.7 1.7) (drill 1.02) (layers "*.Cu" "*.Mask") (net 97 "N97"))
  (pad "41" smd rect (at -2.54 23.9 90) (size 3.5 1.7) (drill (offset -0.9 0)) (layers "F.Cu" "F.Mask") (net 97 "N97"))
  (pad "42" thru_hole rect (at 0 23.9) (size 1.7 1.7) (drill 1.02) (layers "*.Cu" "*.Mask") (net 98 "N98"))
  (pad "42" smd rect (at 0 23.9 90) (size 3.5 1.7) (drill (offset -0.9 0)) (layers "F.Cu" "F.Mask") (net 98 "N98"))
  (pad "43" thru_hole oval (at 2.54 23.9) (size 1.7 1.7) (drill 1.02) (layers "*.Cu" "*.Mask") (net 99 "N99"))
  (pad "43" smd rect (at 2.54 23.9 90) (size 3.5 1.7) (drill (offset -0.9 0)) (layers "F.Cu" "F.Mask") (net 99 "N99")))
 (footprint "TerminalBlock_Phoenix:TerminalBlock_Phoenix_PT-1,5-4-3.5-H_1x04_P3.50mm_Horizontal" (layer "F.Cu") (at 149.16 75.1 90)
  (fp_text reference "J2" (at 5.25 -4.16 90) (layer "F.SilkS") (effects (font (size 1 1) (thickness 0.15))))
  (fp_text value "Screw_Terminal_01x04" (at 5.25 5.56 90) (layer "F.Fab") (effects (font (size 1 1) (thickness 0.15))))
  (pad "1" thru_hole rect (at 0 0 90) (size 2.4 2.4) (drill 1.2) (layers "*.Cu" "*.Mask") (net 1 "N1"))
  (pad "2" thru_hole circle (at 3.5 0 90) (size 2.4 2.4) (drill 1.2) (layers "*.Cu" "*.Mask") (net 2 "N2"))
  (pad "3" thru_hole circle (at 7 0 90) (size 2.4 2.4) (drill 1.2) (layers "*.Cu" "*.Mask") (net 3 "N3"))
  (pad "4" thru_hole circle (at 10.5 0 90) (size 2.4 2.4) (drill 1.2) (layers "*.Cu" "*.Mask") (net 4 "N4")))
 (gr_rect (start 55.88 43.815) (end 208.28 118.745) (stroke (width 0.1) (type default)) (fill none) (layer "Edge.Cuts"))
 (segment (start 149.16 75.1) (end 188.4631 75.1) (width 0.25) (layer "F.Cu") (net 1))
 (segment (start 190.16 74.93) (end 188.6331 74.93) (width 0.25) (layer "F.Cu") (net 1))
 (segment (start 188.4631 75.1) (end 188.6331 74.93) (width 0.25) (layer "F.Cu") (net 1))
 (segment (start 149.33 71.43) (end 149.16 71.6) (width 0.25) (layer "F.Cu") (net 2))
 (segment (start 190.16 71.43) (end 149.33 71.43) (width 0.25) (layer "F.Cu") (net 2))
 (segment (start 149.33 67.93) (end 149.16 68.1) (width 0.25) (layer "F.Cu") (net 3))
 (segment (start 190.16 67.93) (end 149.33 67.93) (width 0.25) (layer "F.Cu") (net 3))
 (segment (start 149.33 64.43) (end 149.16 64.6) (width 0.25) (layer "F.Cu") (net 4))
 (segment (start 190.16 64.43) (end 149.33 64.43) (width 0.25) (layer "F.Cu") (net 4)))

